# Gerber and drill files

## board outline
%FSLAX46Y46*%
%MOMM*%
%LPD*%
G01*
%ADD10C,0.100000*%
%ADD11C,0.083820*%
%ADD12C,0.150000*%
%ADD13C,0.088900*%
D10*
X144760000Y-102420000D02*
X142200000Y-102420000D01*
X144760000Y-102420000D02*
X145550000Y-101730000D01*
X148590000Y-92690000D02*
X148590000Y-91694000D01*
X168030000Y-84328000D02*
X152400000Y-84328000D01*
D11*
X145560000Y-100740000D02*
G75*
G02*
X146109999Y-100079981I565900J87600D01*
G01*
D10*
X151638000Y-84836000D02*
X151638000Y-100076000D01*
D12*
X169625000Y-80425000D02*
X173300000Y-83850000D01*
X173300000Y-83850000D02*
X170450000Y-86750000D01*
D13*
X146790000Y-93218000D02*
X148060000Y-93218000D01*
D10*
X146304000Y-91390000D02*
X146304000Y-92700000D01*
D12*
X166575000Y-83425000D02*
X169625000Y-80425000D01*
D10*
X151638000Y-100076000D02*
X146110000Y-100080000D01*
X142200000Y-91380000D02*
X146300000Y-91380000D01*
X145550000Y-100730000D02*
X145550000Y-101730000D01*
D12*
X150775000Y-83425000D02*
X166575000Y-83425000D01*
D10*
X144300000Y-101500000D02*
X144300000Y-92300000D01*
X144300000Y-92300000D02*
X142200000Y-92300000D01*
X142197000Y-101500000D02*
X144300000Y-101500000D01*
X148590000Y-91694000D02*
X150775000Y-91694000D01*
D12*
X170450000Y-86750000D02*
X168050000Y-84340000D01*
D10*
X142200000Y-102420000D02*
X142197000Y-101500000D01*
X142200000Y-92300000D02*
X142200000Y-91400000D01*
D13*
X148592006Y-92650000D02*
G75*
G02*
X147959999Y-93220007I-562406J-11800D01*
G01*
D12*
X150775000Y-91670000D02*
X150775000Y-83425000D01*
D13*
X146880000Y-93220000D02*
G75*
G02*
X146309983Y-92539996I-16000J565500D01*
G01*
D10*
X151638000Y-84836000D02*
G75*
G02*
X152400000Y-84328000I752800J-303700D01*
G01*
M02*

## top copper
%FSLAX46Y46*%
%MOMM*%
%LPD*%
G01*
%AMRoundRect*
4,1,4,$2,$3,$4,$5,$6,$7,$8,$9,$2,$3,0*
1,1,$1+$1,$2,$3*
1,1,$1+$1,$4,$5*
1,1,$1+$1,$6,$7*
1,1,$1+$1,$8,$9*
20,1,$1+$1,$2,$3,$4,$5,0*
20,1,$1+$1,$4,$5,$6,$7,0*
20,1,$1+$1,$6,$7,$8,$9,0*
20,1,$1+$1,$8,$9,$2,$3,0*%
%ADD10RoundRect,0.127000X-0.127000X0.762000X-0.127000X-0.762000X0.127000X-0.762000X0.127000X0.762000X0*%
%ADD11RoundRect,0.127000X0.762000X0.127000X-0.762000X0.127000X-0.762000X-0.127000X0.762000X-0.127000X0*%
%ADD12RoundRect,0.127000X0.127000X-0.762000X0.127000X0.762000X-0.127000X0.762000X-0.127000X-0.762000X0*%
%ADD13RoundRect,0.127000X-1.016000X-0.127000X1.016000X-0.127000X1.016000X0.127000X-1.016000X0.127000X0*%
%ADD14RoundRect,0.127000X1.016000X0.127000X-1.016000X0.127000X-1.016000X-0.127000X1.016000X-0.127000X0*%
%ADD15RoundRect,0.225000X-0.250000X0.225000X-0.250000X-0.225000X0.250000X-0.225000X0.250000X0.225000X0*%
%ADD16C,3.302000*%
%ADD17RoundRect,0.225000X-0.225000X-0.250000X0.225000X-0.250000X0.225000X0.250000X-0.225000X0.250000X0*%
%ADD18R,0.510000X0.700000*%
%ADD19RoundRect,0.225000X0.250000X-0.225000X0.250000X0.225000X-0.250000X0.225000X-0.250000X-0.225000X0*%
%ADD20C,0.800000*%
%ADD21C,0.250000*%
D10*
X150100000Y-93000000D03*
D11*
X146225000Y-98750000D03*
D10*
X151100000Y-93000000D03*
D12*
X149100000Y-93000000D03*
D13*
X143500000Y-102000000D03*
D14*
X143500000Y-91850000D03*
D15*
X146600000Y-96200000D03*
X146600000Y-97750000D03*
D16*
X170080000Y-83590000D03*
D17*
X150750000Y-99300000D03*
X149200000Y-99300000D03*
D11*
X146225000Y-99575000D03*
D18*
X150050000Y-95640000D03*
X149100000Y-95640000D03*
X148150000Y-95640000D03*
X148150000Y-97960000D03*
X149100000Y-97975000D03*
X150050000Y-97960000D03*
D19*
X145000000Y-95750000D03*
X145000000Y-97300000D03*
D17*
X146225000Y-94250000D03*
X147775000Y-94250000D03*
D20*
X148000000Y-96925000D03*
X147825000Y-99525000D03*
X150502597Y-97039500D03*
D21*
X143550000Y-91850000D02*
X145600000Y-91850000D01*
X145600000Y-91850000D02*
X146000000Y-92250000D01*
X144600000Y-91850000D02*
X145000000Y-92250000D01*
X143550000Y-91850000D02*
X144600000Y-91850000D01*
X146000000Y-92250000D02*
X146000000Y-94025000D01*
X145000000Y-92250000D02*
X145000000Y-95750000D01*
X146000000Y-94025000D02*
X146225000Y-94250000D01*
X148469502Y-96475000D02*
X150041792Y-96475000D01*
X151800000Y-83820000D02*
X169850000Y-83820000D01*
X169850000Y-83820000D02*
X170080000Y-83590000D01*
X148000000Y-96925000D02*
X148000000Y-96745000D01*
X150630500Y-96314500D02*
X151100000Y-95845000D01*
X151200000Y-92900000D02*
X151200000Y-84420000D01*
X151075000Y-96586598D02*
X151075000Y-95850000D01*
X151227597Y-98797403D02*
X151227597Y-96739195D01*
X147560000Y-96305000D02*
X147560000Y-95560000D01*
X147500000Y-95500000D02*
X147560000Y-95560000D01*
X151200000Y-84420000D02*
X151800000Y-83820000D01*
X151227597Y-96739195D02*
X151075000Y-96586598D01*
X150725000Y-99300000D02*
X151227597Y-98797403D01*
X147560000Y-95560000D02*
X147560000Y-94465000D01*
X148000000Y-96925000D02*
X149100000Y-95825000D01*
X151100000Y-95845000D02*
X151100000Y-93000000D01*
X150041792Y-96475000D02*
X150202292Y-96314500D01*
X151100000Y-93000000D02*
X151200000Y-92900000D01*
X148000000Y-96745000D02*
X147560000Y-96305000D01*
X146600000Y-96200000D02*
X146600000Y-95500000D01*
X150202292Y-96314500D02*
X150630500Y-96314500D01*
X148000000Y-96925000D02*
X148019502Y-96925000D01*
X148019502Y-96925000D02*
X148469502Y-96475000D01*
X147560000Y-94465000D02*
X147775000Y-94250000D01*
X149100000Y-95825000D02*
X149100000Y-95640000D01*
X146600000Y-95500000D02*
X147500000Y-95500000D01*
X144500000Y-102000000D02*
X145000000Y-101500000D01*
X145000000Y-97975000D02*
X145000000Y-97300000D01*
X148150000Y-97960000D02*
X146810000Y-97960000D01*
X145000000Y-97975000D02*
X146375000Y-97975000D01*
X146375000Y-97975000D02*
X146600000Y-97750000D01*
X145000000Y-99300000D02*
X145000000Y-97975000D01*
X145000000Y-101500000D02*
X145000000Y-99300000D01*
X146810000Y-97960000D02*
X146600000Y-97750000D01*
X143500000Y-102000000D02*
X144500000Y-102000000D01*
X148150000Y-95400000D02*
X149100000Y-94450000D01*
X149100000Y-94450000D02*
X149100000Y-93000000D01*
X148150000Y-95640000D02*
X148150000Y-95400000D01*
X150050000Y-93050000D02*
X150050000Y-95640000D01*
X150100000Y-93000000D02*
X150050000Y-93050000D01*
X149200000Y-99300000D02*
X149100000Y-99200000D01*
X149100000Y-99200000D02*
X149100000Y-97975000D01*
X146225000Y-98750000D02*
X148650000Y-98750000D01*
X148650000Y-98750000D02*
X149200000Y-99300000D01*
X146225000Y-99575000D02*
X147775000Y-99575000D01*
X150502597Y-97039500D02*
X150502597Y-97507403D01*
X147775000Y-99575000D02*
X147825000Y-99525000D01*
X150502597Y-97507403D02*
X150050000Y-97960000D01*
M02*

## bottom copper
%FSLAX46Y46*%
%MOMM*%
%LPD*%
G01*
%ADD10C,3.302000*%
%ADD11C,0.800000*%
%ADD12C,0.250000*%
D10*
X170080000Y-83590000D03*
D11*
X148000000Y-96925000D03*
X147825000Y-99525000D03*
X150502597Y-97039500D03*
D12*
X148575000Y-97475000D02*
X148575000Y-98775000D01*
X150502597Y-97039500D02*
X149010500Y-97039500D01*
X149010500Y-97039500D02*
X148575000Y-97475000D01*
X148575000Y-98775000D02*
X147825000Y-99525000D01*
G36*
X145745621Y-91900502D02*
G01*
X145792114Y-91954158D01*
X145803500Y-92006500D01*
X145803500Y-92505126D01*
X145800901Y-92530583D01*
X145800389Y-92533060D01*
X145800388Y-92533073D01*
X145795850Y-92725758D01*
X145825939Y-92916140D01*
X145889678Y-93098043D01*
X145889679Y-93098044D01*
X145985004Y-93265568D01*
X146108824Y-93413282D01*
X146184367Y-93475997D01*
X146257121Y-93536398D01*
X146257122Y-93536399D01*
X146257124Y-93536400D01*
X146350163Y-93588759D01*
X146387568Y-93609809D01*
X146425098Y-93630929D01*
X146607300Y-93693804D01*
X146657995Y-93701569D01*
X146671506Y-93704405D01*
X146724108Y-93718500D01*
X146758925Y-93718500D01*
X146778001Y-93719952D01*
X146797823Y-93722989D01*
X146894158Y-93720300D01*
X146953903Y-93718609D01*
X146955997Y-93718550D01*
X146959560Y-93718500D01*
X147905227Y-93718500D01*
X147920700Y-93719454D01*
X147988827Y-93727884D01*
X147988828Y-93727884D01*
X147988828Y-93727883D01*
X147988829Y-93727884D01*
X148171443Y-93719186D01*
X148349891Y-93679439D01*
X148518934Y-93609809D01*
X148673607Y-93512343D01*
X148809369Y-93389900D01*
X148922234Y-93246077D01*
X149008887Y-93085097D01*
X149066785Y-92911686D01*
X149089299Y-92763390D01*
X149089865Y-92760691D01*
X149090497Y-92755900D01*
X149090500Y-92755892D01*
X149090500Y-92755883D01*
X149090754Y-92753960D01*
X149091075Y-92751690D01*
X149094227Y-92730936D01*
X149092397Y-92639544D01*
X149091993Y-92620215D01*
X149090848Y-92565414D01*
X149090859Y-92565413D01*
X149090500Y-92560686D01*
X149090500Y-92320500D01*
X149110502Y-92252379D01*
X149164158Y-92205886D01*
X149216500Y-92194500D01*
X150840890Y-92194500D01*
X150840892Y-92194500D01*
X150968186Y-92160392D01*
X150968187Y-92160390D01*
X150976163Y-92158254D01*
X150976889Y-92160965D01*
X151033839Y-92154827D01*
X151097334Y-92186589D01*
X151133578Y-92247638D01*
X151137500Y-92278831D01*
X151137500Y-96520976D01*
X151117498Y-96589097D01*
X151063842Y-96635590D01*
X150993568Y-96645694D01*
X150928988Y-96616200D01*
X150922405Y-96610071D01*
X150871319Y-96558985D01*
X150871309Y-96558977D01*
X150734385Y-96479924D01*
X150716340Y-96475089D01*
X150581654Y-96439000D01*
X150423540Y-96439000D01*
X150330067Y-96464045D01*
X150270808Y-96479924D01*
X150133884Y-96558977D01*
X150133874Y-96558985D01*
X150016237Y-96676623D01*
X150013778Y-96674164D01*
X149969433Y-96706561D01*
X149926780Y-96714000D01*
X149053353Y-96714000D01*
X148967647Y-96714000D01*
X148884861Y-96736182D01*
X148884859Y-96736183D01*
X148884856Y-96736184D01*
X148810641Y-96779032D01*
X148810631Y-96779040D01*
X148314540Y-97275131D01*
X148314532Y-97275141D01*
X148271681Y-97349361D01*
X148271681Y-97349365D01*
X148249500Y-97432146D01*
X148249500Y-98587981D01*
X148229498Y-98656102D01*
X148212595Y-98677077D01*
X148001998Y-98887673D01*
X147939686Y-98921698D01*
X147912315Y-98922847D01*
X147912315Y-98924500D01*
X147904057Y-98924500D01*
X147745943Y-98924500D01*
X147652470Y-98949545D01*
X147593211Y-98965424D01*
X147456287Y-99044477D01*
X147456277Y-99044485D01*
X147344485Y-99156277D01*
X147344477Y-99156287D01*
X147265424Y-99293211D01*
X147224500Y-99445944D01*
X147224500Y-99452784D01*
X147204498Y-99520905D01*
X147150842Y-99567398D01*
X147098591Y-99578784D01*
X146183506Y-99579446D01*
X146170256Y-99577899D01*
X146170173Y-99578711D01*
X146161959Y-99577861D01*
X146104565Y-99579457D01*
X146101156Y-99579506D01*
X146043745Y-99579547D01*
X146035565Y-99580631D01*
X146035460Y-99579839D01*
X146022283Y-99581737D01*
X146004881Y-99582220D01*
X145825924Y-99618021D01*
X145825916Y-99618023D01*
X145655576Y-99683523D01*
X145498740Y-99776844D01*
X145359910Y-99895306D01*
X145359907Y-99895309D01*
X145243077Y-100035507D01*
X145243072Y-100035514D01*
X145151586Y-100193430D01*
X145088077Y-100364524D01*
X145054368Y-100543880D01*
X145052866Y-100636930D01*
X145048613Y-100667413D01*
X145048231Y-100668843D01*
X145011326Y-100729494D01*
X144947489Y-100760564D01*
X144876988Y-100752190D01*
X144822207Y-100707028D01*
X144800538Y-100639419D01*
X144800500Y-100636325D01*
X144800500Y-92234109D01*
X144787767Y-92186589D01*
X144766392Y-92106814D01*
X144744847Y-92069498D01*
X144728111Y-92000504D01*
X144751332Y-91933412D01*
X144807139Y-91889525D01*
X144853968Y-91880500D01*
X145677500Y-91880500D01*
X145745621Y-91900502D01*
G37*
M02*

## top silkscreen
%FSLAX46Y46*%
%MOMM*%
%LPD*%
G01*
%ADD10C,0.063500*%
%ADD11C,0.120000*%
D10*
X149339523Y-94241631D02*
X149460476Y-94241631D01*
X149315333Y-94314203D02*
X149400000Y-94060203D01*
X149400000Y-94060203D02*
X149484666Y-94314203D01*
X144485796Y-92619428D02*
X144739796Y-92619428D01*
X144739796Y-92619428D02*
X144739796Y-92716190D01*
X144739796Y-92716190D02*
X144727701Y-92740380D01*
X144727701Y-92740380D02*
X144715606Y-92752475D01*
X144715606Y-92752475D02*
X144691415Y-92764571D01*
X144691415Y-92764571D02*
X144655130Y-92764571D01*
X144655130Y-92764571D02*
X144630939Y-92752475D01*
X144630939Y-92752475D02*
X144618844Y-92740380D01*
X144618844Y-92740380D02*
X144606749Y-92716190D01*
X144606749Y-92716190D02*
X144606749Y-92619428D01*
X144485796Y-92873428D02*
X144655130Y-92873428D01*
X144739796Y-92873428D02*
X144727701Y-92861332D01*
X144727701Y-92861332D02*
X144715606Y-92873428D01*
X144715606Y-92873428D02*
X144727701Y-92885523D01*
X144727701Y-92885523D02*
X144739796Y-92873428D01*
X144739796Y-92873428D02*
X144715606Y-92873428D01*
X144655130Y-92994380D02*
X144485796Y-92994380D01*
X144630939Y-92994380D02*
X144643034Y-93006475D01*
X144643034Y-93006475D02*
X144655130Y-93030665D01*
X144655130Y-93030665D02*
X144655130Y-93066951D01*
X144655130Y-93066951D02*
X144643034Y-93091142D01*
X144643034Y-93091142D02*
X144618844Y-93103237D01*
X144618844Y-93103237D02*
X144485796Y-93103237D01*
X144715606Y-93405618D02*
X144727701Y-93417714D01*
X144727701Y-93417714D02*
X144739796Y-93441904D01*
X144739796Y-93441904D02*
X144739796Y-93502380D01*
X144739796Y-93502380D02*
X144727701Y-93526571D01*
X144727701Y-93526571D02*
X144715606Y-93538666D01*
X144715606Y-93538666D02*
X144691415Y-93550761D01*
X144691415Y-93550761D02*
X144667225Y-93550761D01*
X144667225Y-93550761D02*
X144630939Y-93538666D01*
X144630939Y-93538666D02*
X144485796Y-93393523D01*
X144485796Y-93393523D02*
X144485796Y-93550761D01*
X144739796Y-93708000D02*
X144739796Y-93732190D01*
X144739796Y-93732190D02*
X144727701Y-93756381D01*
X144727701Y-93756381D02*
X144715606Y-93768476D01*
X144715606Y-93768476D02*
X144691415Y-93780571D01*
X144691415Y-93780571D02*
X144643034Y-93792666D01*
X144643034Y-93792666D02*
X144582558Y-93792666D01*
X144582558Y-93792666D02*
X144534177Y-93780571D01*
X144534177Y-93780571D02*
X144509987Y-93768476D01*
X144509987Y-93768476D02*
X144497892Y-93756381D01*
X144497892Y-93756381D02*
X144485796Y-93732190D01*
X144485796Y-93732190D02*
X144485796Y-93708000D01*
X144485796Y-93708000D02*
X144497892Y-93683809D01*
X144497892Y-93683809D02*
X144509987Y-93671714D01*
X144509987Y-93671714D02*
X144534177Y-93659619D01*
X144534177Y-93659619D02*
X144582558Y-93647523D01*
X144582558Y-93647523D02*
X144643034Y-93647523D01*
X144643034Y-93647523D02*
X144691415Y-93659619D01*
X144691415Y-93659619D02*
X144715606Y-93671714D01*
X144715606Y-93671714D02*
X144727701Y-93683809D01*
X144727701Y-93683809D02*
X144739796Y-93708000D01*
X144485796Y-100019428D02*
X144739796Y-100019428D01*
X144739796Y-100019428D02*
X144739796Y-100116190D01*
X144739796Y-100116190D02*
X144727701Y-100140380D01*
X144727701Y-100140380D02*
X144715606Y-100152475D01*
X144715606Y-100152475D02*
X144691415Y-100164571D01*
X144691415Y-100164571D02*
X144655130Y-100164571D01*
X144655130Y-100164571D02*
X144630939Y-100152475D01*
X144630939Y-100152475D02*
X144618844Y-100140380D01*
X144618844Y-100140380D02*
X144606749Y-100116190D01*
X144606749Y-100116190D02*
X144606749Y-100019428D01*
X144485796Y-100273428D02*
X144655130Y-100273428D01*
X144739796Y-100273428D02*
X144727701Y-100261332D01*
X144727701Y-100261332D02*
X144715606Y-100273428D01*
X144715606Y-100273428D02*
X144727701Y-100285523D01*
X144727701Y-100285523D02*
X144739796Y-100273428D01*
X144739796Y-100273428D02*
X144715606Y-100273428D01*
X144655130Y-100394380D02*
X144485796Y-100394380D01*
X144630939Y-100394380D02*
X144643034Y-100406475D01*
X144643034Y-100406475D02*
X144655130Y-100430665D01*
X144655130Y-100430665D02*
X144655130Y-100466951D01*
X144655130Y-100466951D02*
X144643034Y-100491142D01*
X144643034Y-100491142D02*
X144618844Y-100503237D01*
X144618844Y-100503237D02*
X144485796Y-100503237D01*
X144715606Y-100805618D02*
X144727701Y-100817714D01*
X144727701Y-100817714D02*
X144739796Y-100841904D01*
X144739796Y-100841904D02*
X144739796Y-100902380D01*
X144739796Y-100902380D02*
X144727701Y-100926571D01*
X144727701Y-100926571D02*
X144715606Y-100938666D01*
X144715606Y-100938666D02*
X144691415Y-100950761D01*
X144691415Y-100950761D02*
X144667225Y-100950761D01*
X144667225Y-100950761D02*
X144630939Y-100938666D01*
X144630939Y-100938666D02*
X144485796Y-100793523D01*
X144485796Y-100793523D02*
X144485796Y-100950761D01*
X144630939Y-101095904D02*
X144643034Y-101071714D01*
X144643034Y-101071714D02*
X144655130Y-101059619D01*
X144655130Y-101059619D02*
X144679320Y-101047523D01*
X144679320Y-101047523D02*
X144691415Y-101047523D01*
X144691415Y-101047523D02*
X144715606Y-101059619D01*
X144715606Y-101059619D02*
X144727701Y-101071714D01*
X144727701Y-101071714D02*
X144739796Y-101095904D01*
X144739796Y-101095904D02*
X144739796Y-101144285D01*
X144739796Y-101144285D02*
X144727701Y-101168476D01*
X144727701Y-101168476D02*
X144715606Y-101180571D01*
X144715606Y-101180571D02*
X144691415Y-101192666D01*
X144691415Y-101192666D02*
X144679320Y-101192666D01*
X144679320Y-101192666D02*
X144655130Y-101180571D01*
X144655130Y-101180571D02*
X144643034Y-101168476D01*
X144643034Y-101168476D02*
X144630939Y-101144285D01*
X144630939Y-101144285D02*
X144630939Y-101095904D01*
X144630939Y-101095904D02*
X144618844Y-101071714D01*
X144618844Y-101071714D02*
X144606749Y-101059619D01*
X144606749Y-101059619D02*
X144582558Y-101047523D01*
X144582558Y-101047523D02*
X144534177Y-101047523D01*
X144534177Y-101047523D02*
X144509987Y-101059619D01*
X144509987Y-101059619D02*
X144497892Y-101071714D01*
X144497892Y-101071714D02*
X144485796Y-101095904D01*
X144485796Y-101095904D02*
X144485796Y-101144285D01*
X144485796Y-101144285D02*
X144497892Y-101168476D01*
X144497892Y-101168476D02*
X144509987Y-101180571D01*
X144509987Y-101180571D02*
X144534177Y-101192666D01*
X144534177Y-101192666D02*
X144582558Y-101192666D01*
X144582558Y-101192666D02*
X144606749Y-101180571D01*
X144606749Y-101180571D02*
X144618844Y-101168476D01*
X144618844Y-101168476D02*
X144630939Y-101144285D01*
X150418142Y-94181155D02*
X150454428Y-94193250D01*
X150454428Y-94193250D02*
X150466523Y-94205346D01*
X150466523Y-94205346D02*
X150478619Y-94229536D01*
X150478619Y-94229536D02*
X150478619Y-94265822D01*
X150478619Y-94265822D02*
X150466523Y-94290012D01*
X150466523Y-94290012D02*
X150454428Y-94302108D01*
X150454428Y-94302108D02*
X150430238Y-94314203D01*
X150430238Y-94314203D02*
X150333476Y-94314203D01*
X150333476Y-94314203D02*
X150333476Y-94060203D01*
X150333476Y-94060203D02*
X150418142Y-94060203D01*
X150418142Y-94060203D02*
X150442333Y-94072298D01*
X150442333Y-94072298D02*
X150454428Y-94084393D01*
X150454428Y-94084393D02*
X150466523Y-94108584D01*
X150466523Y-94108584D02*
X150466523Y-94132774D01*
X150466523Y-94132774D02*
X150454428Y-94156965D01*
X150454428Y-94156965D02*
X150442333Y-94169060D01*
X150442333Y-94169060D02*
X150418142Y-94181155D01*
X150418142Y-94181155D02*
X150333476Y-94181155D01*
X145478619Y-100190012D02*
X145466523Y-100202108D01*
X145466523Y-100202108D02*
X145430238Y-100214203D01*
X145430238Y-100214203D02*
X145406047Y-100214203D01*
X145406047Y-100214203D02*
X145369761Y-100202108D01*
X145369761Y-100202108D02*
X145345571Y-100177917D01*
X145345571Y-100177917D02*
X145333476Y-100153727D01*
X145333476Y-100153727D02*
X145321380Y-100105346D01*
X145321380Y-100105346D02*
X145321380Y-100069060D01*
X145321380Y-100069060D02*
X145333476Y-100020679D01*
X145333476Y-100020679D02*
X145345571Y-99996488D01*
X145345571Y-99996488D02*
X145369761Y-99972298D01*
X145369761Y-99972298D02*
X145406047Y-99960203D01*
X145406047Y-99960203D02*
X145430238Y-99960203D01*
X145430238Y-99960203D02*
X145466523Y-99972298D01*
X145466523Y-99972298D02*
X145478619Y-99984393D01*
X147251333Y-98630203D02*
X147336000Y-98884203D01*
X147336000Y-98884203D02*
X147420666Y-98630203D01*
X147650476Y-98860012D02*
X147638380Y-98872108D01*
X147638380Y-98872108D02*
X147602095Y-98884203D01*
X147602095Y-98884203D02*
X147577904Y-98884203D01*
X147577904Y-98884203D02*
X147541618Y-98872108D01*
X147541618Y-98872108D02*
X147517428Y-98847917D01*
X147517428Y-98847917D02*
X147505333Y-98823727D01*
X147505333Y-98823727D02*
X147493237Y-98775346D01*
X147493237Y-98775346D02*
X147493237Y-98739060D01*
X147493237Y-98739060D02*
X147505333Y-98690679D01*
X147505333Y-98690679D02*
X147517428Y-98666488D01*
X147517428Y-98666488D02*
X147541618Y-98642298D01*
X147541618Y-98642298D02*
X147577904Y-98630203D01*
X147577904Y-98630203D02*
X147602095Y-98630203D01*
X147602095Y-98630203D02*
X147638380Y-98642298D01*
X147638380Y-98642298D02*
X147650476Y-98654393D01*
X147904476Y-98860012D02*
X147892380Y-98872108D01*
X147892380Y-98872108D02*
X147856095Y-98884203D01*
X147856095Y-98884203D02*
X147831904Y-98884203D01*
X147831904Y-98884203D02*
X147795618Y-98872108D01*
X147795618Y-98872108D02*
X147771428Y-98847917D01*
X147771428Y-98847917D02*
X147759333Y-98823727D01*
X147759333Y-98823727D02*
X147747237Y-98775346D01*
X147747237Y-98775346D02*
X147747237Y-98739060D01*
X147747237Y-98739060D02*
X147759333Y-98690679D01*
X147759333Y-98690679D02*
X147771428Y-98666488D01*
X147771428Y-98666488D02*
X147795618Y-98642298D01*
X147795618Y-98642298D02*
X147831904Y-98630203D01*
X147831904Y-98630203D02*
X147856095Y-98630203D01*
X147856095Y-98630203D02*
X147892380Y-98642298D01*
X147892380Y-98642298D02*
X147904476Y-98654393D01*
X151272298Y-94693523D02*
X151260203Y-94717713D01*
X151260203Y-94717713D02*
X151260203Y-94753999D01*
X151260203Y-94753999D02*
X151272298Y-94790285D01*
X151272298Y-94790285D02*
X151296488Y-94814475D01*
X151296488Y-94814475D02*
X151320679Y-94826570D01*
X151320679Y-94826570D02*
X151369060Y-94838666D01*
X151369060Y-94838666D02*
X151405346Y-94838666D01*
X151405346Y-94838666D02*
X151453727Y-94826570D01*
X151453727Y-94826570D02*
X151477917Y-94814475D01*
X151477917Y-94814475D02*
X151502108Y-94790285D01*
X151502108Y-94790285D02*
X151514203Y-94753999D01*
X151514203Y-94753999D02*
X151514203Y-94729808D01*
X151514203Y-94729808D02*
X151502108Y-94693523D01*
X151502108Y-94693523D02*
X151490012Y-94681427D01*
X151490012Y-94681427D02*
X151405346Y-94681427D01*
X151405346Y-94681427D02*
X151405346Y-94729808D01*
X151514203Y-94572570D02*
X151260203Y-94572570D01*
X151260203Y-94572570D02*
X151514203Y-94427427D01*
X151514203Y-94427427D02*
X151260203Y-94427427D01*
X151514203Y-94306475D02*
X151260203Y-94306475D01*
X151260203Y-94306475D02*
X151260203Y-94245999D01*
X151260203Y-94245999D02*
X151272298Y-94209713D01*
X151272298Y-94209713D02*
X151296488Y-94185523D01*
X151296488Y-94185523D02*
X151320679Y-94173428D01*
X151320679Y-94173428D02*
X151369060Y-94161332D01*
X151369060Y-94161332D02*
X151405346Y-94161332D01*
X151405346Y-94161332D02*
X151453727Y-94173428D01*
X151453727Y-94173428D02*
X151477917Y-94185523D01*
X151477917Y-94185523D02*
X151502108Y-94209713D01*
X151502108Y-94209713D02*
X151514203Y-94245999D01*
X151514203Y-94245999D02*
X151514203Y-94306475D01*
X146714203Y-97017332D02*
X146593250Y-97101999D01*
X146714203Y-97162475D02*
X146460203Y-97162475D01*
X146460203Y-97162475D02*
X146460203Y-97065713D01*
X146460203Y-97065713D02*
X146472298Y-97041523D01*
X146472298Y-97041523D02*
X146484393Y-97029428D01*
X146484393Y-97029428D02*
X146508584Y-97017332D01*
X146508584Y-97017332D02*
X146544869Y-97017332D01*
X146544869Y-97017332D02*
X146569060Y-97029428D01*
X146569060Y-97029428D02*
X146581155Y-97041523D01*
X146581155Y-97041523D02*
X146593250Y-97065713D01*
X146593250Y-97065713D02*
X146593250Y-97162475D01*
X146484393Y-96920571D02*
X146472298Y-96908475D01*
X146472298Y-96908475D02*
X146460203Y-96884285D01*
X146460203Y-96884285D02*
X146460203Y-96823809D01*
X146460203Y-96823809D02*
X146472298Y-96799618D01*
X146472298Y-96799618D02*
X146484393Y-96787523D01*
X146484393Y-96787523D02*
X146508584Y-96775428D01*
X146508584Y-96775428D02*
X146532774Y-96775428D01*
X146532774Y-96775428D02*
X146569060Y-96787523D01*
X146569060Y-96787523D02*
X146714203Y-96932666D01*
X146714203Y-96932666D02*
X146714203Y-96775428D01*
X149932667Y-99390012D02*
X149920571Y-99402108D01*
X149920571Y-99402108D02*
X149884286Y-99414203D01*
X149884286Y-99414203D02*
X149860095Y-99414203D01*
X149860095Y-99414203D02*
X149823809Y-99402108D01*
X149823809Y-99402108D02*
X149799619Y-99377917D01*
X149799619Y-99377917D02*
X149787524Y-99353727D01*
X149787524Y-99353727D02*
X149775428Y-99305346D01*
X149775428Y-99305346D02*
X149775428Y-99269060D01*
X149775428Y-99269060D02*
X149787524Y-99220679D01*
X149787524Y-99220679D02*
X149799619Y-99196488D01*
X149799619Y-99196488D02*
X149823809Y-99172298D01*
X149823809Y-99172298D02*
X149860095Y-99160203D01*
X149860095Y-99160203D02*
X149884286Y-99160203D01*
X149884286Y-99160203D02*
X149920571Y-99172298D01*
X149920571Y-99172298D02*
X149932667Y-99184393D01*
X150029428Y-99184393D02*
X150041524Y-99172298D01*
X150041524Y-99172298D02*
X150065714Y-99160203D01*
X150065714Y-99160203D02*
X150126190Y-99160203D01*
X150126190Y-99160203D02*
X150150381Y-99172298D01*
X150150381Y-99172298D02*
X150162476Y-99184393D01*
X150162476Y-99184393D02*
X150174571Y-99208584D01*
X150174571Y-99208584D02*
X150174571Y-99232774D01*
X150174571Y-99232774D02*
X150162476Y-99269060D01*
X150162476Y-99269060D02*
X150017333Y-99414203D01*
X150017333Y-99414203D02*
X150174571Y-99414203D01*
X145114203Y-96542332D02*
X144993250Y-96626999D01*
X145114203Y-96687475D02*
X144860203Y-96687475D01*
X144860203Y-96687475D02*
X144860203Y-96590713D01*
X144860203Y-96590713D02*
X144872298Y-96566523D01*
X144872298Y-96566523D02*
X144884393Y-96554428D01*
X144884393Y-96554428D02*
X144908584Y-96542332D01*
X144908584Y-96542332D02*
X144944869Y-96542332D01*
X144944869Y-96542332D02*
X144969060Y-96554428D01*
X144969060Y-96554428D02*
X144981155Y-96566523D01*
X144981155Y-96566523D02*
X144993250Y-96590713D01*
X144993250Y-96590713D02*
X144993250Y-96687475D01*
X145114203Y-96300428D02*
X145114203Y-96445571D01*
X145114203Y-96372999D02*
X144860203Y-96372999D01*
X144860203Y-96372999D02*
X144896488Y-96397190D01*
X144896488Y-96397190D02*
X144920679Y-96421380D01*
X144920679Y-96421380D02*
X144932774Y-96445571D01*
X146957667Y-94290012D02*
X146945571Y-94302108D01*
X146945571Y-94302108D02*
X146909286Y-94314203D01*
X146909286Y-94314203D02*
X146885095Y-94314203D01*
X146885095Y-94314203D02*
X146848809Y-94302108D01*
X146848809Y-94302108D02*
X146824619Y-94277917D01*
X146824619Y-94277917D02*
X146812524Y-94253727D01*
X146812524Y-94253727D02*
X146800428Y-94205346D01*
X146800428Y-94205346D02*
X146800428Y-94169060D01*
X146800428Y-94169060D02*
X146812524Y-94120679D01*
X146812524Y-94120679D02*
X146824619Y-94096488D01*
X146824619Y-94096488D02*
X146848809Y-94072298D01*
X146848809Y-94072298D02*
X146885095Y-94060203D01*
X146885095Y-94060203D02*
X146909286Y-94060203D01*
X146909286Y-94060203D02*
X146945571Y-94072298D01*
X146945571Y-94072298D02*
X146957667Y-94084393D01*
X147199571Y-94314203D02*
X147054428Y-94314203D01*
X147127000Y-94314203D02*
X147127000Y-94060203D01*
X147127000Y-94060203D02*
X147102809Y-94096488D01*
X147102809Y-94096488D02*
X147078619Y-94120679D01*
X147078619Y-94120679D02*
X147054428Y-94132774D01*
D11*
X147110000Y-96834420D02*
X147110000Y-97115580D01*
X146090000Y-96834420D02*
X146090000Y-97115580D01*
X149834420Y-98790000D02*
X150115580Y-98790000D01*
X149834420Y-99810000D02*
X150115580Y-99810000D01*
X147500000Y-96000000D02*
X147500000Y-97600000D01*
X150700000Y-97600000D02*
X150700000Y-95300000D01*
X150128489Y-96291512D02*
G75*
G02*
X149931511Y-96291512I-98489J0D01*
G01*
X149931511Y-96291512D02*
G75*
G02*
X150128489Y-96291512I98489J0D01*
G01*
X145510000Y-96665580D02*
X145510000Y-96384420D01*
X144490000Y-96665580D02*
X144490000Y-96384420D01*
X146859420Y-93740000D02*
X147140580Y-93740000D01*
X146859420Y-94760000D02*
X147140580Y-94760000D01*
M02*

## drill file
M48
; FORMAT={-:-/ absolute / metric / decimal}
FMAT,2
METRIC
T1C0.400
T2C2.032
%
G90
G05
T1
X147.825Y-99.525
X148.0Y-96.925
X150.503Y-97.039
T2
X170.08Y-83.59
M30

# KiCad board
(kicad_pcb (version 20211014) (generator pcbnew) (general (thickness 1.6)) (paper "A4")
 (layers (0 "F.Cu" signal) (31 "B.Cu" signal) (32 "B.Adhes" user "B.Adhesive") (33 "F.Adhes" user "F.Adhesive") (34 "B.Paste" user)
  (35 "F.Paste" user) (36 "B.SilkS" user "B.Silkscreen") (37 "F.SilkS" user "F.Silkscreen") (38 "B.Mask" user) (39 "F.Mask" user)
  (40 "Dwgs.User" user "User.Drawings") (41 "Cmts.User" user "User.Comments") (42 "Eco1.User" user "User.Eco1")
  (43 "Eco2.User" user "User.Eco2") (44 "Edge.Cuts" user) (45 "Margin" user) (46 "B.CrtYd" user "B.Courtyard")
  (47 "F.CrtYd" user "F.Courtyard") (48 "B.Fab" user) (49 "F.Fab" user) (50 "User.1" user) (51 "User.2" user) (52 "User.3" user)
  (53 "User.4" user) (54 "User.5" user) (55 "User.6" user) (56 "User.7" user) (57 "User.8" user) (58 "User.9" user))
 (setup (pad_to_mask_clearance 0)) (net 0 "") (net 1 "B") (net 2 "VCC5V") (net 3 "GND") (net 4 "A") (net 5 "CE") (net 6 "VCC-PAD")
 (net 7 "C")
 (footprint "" (layer "F.Cu") (at 150.1 93 90)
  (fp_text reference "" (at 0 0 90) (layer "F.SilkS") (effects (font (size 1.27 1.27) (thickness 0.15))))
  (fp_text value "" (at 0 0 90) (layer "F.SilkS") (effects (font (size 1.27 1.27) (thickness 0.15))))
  (pad "10" smd roundrect (at 0 0 270) (size 1.778 0.508) (layers "F.Cu" "F.Paste" "F.Mask") (roundrect_rratio 0.25) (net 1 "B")))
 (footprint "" (layer "F.Cu") (at 146.225 98.75 -90)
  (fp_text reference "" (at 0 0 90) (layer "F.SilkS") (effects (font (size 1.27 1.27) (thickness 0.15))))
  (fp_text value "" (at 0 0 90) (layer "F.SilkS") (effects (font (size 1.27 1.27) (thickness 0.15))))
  (pad "B" smd roundrect (at 0 0 180) (size 1.778 0.508) (layers "F.Cu" "F.Paste" "F.Mask") (roundrect_rratio 0.25) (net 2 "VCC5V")))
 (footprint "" (layer "F.Cu") (at 151.1 93 90)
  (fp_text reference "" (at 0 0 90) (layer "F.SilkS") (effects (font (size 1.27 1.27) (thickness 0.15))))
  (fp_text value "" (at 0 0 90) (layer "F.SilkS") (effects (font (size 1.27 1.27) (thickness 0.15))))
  (pad "9" smd roundrect (at 0 0 270) (size 1.778 0.508) (layers "F.Cu" "F.Paste" "F.Mask") (roundrect_rratio 0.25) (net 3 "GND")))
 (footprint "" (layer "F.Cu") (at 149.1 93 -90)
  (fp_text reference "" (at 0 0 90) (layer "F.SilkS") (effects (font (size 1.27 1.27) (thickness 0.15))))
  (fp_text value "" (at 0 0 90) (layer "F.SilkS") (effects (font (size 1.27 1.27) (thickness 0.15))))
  (pad "11" smd roundrect (at 0 0 90) (size 1.778 0.508) (layers "F.Cu" "F.Paste" "F.Mask") (roundrect_rratio 0.25) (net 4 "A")))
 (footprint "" (layer "F.Cu") (at 143.5 102)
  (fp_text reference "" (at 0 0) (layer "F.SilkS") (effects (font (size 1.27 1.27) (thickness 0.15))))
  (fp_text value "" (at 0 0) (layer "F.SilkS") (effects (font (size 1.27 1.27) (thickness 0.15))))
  (pad "4" smd roundrect (at 0 0) (size 2.286 0.508) (layers "F.Cu" "F.Paste" "F.Mask") (roundrect_rratio 0.25) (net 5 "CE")))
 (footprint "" (layer "F.Cu") (at 143.5 91.85 180)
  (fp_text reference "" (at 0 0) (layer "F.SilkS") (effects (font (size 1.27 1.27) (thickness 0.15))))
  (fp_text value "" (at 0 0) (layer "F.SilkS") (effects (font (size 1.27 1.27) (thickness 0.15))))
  (pad "1" smd roundrect (at 0 0 180) (size 2.286 0.508) (layers "F.Cu" "F.Paste" "F.Mask") (roundrect_rratio 0.25) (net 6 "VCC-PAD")))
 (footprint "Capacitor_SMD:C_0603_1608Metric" (layer "F.Cu") (at 146.6 96.975 -90)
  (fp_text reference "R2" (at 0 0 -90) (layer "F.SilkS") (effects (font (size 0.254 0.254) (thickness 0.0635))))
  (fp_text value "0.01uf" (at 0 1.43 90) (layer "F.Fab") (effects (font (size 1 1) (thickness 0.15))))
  (fp_line (start -0.14058 -0.51) (end 0.14058 -0.51) (layer "F.SilkS") (width 0.12))
  (fp_line (start -0.14058 0.51) (end 0.14058 0.51) (layer "F.SilkS") (width 0.12))
  (pad "5" smd roundrect (at -0.775 0 270) (size 0.9 0.95) (layers "F.Cu" "F.Paste" "F.Mask") (roundrect_rratio 0.25) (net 3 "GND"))
  (pad "6" smd roundrect (at 0.775 0 270) (size 0.9 0.95) (layers "F.Cu" "F.Paste" "F.Mask") (roundrect_rratio 0.25) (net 5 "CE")))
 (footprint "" (layer "F.Cu") (at 170.08 83.59)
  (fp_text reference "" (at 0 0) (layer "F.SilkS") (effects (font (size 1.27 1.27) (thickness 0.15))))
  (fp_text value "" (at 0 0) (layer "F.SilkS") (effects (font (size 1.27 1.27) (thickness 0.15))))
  (pad "9" thru_hole circle (at 0 0 270) (size 3.302 3.302) (drill 2.032) (layers *.Cu *.Mask) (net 3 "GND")))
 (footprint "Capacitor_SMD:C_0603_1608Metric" (layer "F.Cu") (at 149.975 99.3)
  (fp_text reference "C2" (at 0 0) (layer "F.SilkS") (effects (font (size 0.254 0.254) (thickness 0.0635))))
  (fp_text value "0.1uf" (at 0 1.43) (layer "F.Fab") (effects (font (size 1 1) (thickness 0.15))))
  (fp_line (start -0.14058 -0.51) (end 0.14058 -0.51) (layer "F.SilkS") (width 0.12))
  (fp_line (start -0.14058 0.51) (end 0.14058 0.51) (layer "F.SilkS") (width 0.12))
  (pad "7" smd roundrect (at 0.775 0) (size 0.9 0.95) (layers "F.Cu" "F.Paste" "F.Mask") (roundrect_rratio 0.25) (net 3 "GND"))
  (pad "8" smd roundrect (at -0.775 0) (size 0.9 0.95) (layers "F.Cu" "F.Paste" "F.Mask") (roundrect_rratio 0.25) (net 2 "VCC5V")))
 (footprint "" (layer "F.Cu") (at 146.225 99.575)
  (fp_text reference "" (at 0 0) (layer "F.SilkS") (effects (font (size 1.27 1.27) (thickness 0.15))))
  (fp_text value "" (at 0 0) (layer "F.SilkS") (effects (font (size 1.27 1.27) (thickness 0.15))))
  (pad "B" smd roundrect (at 0 0 180) (size 1.778 0.508) (layers "F.Cu" "F.Paste" "F.Mask") (roundrect_rratio 0.25) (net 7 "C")))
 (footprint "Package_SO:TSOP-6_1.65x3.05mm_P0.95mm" (layer "F.Cu") (at 149.1 96.8 -90)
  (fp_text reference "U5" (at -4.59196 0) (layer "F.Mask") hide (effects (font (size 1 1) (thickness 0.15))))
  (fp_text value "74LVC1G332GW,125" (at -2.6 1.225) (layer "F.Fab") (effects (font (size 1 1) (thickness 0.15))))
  (fp_line (start -0.8 1.6) (end 0.8 1.6) (layer "F.SilkS") (width 0.12))
  (fp_line (start 0.8 -1.6) (end -1.5 -1.6) (layer "F.SilkS") (width 0.12))
  (fp_circle (center -0.508488 -0.93) (end -0.418488 -0.89) (layer "F.SilkS") (width 0.12) (fill none))
  (pad "1" smd rect (at -1.16 -0.95 270) (size 0.7 0.51) (layers "F.Cu" "F.Paste" "F.Mask") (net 1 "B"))
  (pad "2" smd rect (at -1.16 0 270) (size 0.7 0.51) (layers "F.Cu" "F.Paste" "F.Mask") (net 3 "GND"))
  (pad "3" smd rect (at -1.16 0.95 270) (size 0.7 0.51) (layers "F.Cu" "F.Paste" "F.Mask") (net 4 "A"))
  (pad "4" smd rect (at 1.16 0.95 270) (size 0.7 0.51) (layers "F.Cu" "F.Paste" "F.Mask") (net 5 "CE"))
  (pad "5" smd rect (at 1.175 0 270) (size 0.7 0.51) (layers "F.Cu" "F.Paste" "F.Mask") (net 2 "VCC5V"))
  (pad "6" smd rect (at 1.16 -0.95 270) (size 0.7 0.51) (layers "F.Cu" "F.Paste" "F.Mask") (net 7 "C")))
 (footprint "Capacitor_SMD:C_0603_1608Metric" (layer "F.Cu") (at 145 96.525 90)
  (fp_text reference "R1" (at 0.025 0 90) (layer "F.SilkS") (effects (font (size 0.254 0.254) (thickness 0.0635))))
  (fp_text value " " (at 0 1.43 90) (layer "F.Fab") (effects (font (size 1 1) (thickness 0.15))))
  (fp_line (start -0.14058 0.51) (end 0.14058 0.51) (layer "F.SilkS") (width 0.12))
  (fp_line (start -0.14058 -0.51) (end 0.14058 -0.51) (layer "F.SilkS") (width 0.12))
  (pad "2" smd roundrect (at 0.775 0 90) (size 0.9 0.95) (layers "F.Cu" "F.Paste" "F.Mask") (roundrect_rratio 0.25) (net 6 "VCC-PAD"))
  (pad "3" smd roundrect (at -0.775 0 90) (size 0.9 0.95) (layers "F.Cu" "F.Paste" "F.Mask") (roundrect_rratio 0.25) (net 5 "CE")))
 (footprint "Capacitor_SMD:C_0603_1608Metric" (layer "F.Cu") (at 147 94.25)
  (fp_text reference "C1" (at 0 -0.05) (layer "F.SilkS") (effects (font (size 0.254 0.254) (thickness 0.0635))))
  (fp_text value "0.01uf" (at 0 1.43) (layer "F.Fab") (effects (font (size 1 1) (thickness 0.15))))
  (fp_line (start -0.14058 -0.51) (end 0.14058 -0.51) (layer "F.SilkS") (width 0.12))
  (fp_line (start -0.14058 0.51) (end 0.14058 0.51) (layer "F.SilkS") (width 0.12))
  (pad "5" smd roundrect (at -0.775 0) (size 0.9 0.95) (layers "F.Cu" "F.Paste" "F.Mask") (roundrect_rratio 0.25) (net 6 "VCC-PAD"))
  (pad "6" smd roundrect (at 0.775 0) (size 0.9 0.95) (layers "F.Cu" "F.Paste" "F.Mask") (roundrect_rratio 0.25) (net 3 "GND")))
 (gr_line (start 144.76 102.42) (end 142.2 102.42) (layer "Edge.Cuts") (width 0.1))
 (gr_line (start 144.76 102.42) (end 145.55 101.73) (layer "Edge.Cuts") (width 0.1))
 (gr_line (start 148.59 92.69) (end 148.59 91.694) (layer "Edge.Cuts") (width 0.1))
 (gr_line (start 168.03 84.328) (end 152.4 84.328) (layer "Edge.Cuts") (width 0.1))
 (gr_arc (start 145.56 100.74) (mid 145.684497 100.28762) (end 146.11 100.08) (layer "Edge.Cuts") (width 0.08382))
 (gr_line (start 151.638 84.836) (end 151.638 100.076) (layer "Edge.Cuts") (width 0.1))
 (gr_line (start 169.625 80.425) (end 173.3 83.85) (layer "Edge.Cuts") (width 0.15))
 (gr_line (start 173.3 83.85) (end 170.45 86.75) (layer "Edge.Cuts") (width 0.15))
 (gr_line (start 146.79 93.218) (end 148.06 93.218) (layer "Edge.Cuts") (width 0.0889))
 (gr_line (start 146.304 91.39) (end 146.304 92.7) (layer "Edge.Cuts") (width 0.1))
 (gr_line (start 166.575 83.425) (end 169.625 80.425) (layer "Edge.Cuts") (width 0.15))
 (gr_line (start 151.638 100.076) (end 146.11 100.08) (layer "Edge.Cuts") (width 0.1))
 (gr_line (start 142.2 91.38) (end 146.3 91.38) (layer "Edge.Cuts") (width 0.1))
 (gr_line (start 145.55 100.73) (end 145.55 101.73) (layer "Edge.Cuts") (width 0.1))
 (gr_line (start 150.775 83.425) (end 166.575 83.425) (layer "Edge.Cuts") (width 0.15))
 (gr_line (start 144.3 101.5) (end 144.3 92.3) (layer "Edge.Cuts") (width 0.1))
 (gr_line (start 144.3 92.3) (end 142.2 92.3) (layer "Edge.Cuts") (width 0.1))
 (gr_line (start 142.197 101.5) (end 144.3 101.5) (layer "Edge.Cuts") (width 0.1))
 (gr_line (start 148.59 91.694) (end 150.775 91.694) (layer "Edge.Cuts") (width 0.1))
 (gr_line (start 170.45 86.75) (end 168.05 84.34) (layer "Edge.Cuts") (width 0.15))
 (gr_line (start 142.2 102.42) (end 142.197 101.5) (layer "Edge.Cuts") (width 0.1))
 (gr_line (start 142.2 92.3) (end 142.2 91.4) (layer "Edge.Cuts") (width 0.1))
 (gr_arc (start 148.592006 92.65) (mid 148.406336 93.079511) (end 147.96 93.22) (layer "Edge.Cuts") (width 0.0889))
 (gr_line (start 150.775 91.67) (end 150.775 83.425) (layer "Edge.Cuts") (width 0.15))
 (gr_arc (start 146.88 93.22) (mid 146.430454 93.017928) (end 146.31 92.54) (layer "Edge.Cuts") (width 0.0889))
 (gr_arc (start 151.638 84.836) (mid 151.940524 84.464286) (end 152.4 84.328) (layer "Edge.Cuts") (width 0.1))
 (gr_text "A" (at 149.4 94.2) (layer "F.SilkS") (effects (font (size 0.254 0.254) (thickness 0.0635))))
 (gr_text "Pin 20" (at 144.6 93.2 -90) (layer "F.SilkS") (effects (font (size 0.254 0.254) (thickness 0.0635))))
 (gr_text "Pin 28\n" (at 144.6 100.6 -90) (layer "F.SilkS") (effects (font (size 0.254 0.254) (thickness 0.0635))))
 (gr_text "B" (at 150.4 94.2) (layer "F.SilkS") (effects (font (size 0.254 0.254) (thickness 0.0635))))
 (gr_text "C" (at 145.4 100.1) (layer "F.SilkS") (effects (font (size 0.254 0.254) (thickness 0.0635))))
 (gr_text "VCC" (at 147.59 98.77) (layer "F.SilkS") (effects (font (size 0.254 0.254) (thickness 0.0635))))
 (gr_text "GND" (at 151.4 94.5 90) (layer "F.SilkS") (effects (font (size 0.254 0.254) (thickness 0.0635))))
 (segment (start 143.55 91.85) (end 145.6 91.85) (width 0.25) (layer "F.Cu") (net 6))
 (segment (start 145.6 91.85) (end 146 92.25) (width 0.25) (layer "F.Cu") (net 6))
 (segment (start 144.6 91.85) (end 145 92.25) (width 0.25) (layer "F.Cu") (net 6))
 (segment (start 143.55 91.85) (end 144.6 91.85) (width 0.25) (layer "F.Cu") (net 6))
 (segment (start 146 92.25) (end 146 94.025) (width 0.25) (layer "F.Cu") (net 6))
 (segment (start 145 92.25) (end 145 95.75) (width 0.25) (layer "F.Cu") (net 6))
 (segment (start 146 94.025) (end 146.225 94.25) (width 0.25) (layer "F.Cu") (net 6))
 (segment (start 148.469502 96.475) (end 150.041792 96.475) (width 0.25) (layer "F.Cu") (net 3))
 (segment (start 151.8 83.82) (end 169.85 83.82) (width 0.25) (layer "F.Cu") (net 3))
 (segment (start 169.85 83.82) (end 170.08 83.59) (width 0.25) (layer "F.Cu") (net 3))
 (segment (start 148 96.925) (end 148 96.745) (width 0.25) (layer "F.Cu") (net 3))
 (segment (start 150.6305 96.3145) (end 151.1 95.845) (width 0.25) (layer "F.Cu") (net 3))
 (segment (start 151.2 92.9) (end 151.2 84.42) (width 0.25) (layer "F.Cu") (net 3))
 (segment (start 151.075 96.586598) (end 151.075 95.85) (width 0.25) (layer "F.Cu") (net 3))
 (segment (start 151.227597 98.797403) (end 151.227597 96.739195) (width 0.25) (layer "F.Cu") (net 3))
 (segment (start 147.56 96.305) (end 147.56 95.56) (width 0.25) (layer "F.Cu") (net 3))
 (segment (start 147.5 95.5) (end 147.56 95.56) (width 0.25) (layer "F.Cu") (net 3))
 (segment (start 151.2 84.42) (end 151.8 83.82) (width 0.25) (layer "F.Cu") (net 3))
 (segment (start 151.227597 96.739195) (end 151.075 96.586598) (width 0.25) (layer "F.Cu") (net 3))
 (segment (start 150.725 99.3) (end 151.227597 98.797403) (width 0.25) (layer "F.Cu") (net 3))
 (segment (start 147.56 95.56) (end 147.56 94.465) (width 0.25) (layer "F.Cu") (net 3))
 (segment (start 148 96.925) (end 149.1 95.825) (width 0.25) (layer "F.Cu") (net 3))
 (segment (start 151.1 95.845) (end 151.1 93) (width 0.25) (layer "F.Cu") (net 3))
 (segment (start 150.041792 96.475) (end 150.202292 96.3145) (width 0.25) (layer "F.Cu") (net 3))
 (segment (start 151.1 93) (end 151.2 92.9) (width 0.25) (layer "F.Cu") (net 3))
 (segment (start 148 96.745) (end 147.56 96.305) (width 0.25) (layer "F.Cu") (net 3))
 (segment (start 146.6 96.2) (end 146.6 95.5) (width 0.25) (layer "F.Cu") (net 3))
 (segment (start 150.202292 96.3145) (end 150.6305 96.3145) (width 0.25) (layer "F.Cu") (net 3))
 (segment (start 148 96.925) (end 148.019502 96.925) (width 0.25) (layer "F.Cu") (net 3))
 (segment (start 148.019502 96.925) (end 148.469502 96.475) (width 0.25) (layer "F.Cu") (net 3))
 (segment (start 147.56 94.465) (end 147.775 94.25) (width 0.25) (layer "F.Cu") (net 3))
 (segment (start 149.1 95.825) (end 149.1 95.64) (width 0.25) (layer "F.Cu") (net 3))
 (segment (start 146.6 95.5) (end 147.5 95.5) (width 0.25) (layer "F.Cu") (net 3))
 (via (at 148 96.925) (size 0.8) (drill 0.4) (layers "F.Cu" "B.Cu") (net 3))
 (segment (start 144.5 102) (end 145 101.5) (width 0.25) (layer "F.Cu") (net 5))
 (segment (start 145 97.975) (end 145 97.3) (width 0.25) (layer "F.Cu") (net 5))
 (segment (start 148.15 97.96) (end 146.81 97.96) (width 0.25) (layer "F.Cu") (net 5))
 (segment (start 145 97.975) (end 146.375 97.975) (width 0.25) (layer "F.Cu") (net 5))
 (segment (start 146.375 97.975) (end 146.6 97.75) (width 0.25) (layer "F.Cu") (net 5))
 (segment (start 145 99.3) (end 145 97.975) (width 0.25) (layer "F.Cu") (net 5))
 (segment (start 145 101.5) (end 145 99.3) (width 0.25) (layer "F.Cu") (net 5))
 (segment (start 146.81 97.96) (end 146.6 97.75) (width 0.25) (layer "F.Cu") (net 5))
 (segment (start 143.5 102) (end 144.5 102) (width 0.25) (layer "F.Cu") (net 5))
 (segment (start 148.15 95.4) (end 149.1 94.45) (width 0.25) (layer "F.Cu") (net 4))
 (segment (start 149.1 94.45) (end 149.1 93) (width 0.25) (layer "F.Cu") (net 4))
 (segment (start 148.15 95.64) (end 148.15 95.4) (width 0.25) (layer "F.Cu") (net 4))
 (segment (start 150.05 93.05) (end 150.05 95.64) (width 0.25) (layer "F.Cu") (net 1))
 (segment (start 150.1 93) (end 150.05 93.05) (width 0.25) (layer "F.Cu") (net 1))
 (segment (start 149.2 99.3) (end 149.1 99.2) (width 0.25) (layer "F.Cu") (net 2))
 (segment (start 149.1 99.2) (end 149.1 97.975) (width 0.25) (layer "F.Cu") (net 2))
 (segment (start 146.225 98.75) (end 148.65 98.75) (width 0.25) (layer "F.Cu") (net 2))
 (segment (start 148.65 98.75) (end 149.2 99.3) (width 0.25) (layer "F.Cu") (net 2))
 (segment (start 146.225 99.575) (end 147.775 99.575) (width 0.25) (layer "F.Cu") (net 7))
 (segment (start 150.502597 97.0395) (end 150.502597 97.507403) (width 0.25) (layer "F.Cu") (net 7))
 (segment (start 147.775 99.575) (end 147.825 99.525) (width 0.25) (layer "F.Cu") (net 7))
 (segment (start 150.502597 97.507403) (end 150.05 97.96) (width 0.25) (layer "F.Cu") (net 7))
 (via (at 147.825 99.525) (size 0.8) (drill 0.4) (layers "F.Cu" "B.Cu") (free) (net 7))
 (via (at 150.502597 97.0395) (size 0.8) (drill 0.4) (layers "F.Cu" "B.Cu") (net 7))
 (segment (start 148.575 97.475) (end 148.575 98.775) (width 0.25) (layer "B.Cu") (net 7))
 (segment (start 150.502597 97.0395) (end 149.0105 97.0395) (width 0.25) (layer "B.Cu") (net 7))
 (segment (start 149.0105 97.0395) (end 148.575 97.475) (width 0.25) (layer "B.Cu") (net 7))
 (segment (start 148.575 98.775) (end 147.825 99.525) (width 0.25) (layer "B.Cu") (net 7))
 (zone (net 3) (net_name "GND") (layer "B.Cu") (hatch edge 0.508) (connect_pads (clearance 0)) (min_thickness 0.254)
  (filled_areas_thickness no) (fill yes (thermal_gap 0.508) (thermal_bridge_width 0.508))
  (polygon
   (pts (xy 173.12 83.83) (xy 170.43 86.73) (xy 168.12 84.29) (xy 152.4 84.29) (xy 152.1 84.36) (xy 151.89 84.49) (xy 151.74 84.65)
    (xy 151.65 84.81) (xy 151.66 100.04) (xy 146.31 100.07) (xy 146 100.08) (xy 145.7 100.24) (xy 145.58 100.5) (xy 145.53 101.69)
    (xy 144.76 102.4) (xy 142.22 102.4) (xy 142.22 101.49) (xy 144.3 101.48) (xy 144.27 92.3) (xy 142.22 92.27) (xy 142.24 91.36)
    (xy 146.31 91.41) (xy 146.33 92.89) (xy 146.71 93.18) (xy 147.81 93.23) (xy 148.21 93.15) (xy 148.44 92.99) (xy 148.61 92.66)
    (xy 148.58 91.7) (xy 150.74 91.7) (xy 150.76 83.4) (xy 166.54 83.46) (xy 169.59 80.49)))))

